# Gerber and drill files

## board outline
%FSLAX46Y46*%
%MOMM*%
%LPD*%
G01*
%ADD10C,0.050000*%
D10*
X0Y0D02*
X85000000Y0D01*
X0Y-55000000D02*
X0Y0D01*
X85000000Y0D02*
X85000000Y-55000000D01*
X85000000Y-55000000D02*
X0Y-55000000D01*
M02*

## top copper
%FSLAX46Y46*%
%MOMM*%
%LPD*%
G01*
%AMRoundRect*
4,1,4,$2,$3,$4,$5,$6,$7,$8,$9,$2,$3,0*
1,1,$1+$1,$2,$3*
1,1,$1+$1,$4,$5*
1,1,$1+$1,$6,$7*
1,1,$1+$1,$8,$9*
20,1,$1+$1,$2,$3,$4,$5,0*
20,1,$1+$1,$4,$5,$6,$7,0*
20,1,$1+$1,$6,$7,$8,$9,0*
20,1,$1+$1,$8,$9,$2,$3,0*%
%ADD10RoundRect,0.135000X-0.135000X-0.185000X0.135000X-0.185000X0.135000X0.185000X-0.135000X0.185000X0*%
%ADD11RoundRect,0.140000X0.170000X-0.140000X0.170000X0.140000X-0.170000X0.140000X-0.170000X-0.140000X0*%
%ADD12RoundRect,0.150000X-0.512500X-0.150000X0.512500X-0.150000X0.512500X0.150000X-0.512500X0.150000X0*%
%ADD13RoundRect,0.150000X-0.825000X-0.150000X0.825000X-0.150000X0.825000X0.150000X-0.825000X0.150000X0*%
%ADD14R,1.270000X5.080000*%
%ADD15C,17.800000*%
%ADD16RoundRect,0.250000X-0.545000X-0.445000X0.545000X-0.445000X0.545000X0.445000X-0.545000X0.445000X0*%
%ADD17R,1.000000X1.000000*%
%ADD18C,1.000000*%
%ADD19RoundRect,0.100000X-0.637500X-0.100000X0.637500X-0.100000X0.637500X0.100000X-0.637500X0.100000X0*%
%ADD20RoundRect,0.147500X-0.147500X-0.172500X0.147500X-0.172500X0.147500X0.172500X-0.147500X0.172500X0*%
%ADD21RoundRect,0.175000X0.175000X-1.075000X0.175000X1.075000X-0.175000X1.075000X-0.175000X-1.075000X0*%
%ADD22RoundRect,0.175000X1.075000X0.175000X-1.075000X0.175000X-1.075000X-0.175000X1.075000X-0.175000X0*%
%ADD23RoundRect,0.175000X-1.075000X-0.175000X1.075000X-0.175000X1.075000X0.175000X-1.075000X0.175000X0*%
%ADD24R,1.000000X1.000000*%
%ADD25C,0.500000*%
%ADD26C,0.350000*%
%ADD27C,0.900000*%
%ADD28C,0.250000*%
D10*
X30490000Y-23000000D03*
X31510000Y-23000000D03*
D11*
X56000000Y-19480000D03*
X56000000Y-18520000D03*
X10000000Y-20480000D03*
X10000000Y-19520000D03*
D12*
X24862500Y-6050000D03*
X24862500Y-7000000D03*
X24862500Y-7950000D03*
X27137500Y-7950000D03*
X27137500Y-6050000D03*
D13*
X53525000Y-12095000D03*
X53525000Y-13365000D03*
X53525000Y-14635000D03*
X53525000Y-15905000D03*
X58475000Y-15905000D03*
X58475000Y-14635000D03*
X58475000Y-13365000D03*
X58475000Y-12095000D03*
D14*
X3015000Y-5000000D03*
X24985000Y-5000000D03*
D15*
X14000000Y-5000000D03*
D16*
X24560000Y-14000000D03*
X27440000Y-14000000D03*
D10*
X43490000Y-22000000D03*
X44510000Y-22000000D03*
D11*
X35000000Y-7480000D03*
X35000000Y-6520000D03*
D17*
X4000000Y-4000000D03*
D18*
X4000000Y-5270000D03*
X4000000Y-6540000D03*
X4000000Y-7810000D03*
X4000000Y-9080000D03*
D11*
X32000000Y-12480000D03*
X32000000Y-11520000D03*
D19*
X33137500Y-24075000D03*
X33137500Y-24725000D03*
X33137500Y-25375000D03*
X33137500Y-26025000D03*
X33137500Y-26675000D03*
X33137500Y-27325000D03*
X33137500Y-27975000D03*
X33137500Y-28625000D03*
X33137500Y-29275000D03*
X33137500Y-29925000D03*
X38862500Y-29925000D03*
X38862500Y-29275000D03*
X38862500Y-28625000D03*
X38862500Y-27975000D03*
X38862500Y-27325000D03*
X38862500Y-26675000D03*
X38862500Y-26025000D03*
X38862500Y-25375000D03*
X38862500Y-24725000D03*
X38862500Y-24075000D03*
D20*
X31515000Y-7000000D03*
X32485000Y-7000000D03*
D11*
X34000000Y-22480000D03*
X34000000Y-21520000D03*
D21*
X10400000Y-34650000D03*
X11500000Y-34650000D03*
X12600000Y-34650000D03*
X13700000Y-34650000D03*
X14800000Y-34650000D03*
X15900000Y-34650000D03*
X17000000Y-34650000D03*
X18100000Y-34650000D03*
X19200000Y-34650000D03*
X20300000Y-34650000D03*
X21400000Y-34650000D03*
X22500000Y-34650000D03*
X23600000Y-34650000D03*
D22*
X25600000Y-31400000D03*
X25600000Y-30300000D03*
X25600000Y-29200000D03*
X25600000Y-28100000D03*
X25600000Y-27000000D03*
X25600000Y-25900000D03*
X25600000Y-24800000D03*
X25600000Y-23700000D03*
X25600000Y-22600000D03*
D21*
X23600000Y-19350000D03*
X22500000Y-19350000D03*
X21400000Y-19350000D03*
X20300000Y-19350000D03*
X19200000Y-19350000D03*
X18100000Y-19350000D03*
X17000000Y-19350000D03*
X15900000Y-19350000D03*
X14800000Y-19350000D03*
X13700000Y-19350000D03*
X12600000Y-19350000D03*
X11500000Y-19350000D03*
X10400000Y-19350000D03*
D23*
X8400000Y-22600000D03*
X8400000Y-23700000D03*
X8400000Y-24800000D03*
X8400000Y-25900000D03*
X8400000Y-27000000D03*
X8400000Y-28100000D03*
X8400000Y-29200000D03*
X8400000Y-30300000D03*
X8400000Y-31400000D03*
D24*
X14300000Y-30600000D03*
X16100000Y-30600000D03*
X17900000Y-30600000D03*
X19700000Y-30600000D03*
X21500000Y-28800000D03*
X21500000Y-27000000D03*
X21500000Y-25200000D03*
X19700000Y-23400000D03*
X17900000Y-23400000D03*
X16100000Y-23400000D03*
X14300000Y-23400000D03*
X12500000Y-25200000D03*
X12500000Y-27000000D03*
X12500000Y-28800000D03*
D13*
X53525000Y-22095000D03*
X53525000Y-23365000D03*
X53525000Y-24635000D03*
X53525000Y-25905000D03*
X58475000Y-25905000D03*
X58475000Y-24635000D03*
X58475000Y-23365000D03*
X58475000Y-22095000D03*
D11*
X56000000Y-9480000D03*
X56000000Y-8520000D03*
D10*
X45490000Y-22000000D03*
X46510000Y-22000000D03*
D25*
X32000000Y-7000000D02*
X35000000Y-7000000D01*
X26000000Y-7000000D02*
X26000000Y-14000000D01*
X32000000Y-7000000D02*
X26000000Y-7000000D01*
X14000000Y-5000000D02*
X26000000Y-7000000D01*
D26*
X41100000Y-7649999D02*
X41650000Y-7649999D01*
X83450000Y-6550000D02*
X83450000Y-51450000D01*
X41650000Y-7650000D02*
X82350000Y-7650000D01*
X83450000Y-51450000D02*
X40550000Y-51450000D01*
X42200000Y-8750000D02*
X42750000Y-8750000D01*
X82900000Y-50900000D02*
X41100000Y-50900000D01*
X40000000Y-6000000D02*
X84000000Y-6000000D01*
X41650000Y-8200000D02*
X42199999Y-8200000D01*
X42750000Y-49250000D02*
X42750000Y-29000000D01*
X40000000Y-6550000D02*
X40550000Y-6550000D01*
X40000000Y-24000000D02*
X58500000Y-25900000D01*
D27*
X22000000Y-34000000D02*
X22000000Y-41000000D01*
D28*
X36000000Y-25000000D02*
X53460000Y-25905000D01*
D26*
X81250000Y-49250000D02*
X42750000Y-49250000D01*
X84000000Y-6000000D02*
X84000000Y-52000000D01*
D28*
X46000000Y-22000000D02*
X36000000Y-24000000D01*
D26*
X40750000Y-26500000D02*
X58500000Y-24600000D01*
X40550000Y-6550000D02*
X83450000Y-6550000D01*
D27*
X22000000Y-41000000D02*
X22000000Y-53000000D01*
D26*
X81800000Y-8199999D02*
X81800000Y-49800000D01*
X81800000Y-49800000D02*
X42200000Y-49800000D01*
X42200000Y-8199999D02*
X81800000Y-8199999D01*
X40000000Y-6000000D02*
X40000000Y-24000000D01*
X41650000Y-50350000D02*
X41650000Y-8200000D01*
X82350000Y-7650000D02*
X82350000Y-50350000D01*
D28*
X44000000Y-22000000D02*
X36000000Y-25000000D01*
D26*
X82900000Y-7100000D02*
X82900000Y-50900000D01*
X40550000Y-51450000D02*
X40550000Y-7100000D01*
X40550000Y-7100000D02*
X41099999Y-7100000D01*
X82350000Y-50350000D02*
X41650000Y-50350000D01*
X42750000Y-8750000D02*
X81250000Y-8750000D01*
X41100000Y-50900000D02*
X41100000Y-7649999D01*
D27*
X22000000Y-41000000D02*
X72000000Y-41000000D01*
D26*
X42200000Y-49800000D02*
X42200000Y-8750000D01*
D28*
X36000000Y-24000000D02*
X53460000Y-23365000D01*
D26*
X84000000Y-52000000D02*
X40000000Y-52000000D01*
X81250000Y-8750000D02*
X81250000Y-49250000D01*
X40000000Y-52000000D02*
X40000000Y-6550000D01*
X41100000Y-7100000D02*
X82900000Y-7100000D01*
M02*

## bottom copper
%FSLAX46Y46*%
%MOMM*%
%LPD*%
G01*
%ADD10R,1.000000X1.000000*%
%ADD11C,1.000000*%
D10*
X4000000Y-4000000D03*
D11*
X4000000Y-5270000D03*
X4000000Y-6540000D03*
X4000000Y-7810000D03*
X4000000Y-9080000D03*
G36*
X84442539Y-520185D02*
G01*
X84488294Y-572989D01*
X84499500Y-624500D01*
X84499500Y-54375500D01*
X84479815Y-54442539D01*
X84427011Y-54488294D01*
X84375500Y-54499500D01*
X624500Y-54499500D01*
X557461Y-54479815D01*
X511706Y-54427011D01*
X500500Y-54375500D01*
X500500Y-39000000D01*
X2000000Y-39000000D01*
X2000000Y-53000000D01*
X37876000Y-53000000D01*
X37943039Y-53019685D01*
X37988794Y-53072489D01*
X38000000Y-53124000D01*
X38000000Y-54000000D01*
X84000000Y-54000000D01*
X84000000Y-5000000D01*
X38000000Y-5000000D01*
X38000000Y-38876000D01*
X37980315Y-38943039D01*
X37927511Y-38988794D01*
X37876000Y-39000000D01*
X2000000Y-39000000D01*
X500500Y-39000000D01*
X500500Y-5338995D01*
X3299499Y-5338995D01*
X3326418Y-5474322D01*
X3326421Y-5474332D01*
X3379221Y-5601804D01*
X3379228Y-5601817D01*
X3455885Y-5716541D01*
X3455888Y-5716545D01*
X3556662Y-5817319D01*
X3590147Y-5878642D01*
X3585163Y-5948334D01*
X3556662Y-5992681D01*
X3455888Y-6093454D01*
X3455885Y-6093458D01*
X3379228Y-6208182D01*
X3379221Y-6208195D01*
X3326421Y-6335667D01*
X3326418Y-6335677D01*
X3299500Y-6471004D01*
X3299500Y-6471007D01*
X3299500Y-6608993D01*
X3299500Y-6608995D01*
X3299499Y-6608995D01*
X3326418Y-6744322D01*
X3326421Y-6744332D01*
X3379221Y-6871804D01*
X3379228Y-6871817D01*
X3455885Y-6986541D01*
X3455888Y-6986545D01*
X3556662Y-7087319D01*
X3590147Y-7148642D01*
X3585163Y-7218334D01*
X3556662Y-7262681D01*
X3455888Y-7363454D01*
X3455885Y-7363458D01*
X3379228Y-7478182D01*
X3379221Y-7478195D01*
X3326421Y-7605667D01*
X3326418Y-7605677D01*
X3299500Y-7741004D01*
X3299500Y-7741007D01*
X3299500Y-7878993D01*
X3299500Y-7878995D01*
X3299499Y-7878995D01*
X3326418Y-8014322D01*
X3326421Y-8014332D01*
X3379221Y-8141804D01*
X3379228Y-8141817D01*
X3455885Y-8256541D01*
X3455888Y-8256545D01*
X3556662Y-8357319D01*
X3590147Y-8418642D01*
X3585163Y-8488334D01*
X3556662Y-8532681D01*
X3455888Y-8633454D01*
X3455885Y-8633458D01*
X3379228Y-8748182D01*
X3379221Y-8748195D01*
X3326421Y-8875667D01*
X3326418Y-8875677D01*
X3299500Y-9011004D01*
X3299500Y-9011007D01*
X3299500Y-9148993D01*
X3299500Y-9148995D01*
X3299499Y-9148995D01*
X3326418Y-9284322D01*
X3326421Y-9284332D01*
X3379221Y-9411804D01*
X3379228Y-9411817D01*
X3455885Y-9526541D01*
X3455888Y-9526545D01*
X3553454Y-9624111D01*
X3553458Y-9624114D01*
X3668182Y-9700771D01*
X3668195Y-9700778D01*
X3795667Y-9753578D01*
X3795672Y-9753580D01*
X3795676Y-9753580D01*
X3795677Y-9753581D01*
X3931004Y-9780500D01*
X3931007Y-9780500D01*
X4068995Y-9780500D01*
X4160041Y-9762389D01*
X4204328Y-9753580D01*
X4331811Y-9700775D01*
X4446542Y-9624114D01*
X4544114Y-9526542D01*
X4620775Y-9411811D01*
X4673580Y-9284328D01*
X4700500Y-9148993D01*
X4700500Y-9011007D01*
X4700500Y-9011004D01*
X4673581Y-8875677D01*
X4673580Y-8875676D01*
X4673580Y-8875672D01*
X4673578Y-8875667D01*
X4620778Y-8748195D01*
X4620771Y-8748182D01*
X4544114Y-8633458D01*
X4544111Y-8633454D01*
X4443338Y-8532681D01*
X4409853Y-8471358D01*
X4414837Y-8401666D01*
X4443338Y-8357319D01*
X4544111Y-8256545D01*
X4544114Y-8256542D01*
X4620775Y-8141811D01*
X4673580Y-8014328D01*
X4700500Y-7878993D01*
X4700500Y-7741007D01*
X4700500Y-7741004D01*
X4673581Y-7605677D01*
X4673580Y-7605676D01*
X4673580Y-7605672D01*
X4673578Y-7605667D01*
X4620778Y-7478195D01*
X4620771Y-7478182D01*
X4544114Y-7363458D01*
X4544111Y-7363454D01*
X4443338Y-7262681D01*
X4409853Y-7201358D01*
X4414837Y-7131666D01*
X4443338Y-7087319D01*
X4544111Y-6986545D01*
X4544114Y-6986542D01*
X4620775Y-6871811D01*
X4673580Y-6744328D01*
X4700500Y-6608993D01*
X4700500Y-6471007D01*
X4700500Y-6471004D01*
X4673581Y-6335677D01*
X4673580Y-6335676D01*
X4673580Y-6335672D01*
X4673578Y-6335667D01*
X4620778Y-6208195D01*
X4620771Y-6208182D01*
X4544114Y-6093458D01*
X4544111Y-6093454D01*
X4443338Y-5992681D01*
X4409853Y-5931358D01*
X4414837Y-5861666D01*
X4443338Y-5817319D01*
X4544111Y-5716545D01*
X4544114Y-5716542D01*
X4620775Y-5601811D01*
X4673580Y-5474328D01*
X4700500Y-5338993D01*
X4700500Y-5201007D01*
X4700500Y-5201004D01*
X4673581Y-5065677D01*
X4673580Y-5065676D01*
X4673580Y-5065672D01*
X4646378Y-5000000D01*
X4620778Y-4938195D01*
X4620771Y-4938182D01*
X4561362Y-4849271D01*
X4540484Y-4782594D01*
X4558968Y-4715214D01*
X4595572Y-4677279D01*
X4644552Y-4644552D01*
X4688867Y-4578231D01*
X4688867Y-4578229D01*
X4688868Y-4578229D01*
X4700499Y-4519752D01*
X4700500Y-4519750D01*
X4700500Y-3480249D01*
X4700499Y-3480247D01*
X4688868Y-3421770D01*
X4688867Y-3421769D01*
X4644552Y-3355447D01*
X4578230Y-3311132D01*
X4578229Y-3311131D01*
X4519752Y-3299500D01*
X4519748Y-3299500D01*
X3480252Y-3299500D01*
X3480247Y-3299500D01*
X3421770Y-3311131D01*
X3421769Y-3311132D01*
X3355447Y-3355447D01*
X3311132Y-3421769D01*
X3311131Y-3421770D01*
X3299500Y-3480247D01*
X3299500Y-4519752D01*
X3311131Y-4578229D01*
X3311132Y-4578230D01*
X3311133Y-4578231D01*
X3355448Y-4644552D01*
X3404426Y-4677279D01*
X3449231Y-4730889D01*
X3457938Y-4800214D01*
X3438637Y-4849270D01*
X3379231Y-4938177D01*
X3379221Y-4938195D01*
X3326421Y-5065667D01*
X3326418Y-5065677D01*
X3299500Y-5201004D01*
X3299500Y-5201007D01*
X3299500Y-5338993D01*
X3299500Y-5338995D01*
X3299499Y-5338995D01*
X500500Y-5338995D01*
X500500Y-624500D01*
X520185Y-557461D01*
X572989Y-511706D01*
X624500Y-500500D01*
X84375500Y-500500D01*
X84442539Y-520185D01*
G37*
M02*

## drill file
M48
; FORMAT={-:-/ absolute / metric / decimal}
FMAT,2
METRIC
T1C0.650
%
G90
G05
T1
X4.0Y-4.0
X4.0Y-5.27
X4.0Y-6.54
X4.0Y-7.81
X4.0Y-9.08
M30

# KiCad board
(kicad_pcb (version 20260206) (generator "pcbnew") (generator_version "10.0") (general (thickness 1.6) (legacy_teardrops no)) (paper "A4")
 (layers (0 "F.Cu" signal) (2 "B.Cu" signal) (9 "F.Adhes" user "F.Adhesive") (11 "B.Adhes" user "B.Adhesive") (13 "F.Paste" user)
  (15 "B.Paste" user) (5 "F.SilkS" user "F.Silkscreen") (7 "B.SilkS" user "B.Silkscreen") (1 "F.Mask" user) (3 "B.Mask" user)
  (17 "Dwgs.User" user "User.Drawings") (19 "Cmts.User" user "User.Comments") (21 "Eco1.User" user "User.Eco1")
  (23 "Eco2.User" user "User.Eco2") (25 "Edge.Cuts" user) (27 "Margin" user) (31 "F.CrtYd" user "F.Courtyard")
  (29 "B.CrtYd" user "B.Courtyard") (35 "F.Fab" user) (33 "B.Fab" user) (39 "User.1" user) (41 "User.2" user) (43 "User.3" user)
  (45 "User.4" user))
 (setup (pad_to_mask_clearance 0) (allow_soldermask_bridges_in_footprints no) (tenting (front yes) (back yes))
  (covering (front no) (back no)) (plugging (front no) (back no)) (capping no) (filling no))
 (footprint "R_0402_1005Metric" (layer "F.Cu") (at 31 23)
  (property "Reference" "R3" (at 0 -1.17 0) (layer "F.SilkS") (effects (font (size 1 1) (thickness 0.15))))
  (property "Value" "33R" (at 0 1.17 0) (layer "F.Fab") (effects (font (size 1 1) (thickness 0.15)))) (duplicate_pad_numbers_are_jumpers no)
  (pad "1" smd roundrect (at -0.51 0) (size 0.54 0.64) (layers "F.Cu" "F.Mask" "F.Paste") (roundrect_rratio 0.25))
  (pad "2" smd roundrect (at 0.51 0) (size 0.54 0.64) (layers "F.Cu" "F.Mask" "F.Paste") (roundrect_rratio 0.25)))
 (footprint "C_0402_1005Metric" (layer "F.Cu") (at 56 19 90)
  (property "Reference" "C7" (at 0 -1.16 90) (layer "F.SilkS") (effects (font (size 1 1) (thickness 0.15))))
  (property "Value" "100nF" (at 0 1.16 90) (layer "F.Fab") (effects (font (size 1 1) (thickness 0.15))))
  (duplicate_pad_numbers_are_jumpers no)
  (pad "1" smd roundrect (at -0.48 0 90) (size 0.56 0.62) (layers "F.Cu" "F.Mask" "F.Paste") (roundrect_rratio 0.25))
  (pad "2" smd roundrect (at 0.48 0 90) (size 0.56 0.62) (layers "F.Cu" "F.Mask" "F.Paste") (roundrect_rratio 0.25)))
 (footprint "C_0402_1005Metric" (layer "F.Cu") (at 10 20 90)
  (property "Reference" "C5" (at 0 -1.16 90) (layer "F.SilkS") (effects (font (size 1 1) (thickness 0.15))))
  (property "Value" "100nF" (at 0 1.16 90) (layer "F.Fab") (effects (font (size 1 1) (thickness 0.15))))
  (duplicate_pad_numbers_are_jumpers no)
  (pad "1" smd roundrect (at -0.48 0 90) (size 0.56 0.62) (layers "F.Cu" "F.Mask" "F.Paste") (roundrect_rratio 0.25))
  (pad "2" smd roundrect (at 0.48 0 90) (size 0.56 0.62) (layers "F.Cu" "F.Mask" "F.Paste") (roundrect_rratio 0.25)))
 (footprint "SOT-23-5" (layer "F.Cu") (at 26 7)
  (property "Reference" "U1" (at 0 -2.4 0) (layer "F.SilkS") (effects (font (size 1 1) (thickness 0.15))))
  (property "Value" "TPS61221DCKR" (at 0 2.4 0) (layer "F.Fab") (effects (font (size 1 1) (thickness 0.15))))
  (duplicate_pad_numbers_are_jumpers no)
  (pad "1" smd roundrect (at -1.1375 -0.95) (size 1.325 0.6) (layers "F.Cu" "F.Mask" "F.Paste") (roundrect_rratio 0.25))
  (pad "2" smd roundrect (at -1.1375 0) (size 1.325 0.6) (layers "F.Cu" "F.Mask" "F.Paste") (roundrect_rratio 0.25))
  (pad "3" smd roundrect (at -1.1375 0.95) (size 1.325 0.6) (layers "F.Cu" "F.Mask" "F.Paste") (roundrect_rratio 0.25))
  (pad "4" smd roundrect (at 1.1375 0.95) (size 1.325 0.6) (layers "F.Cu" "F.Mask" "F.Paste") (roundrect_rratio 0.25))
  (pad "5" smd roundrect (at 1.1375 -0.95) (size 1.325 0.6) (layers "F.Cu" "F.Mask" "F.Paste") (roundrect_rratio 0.25)))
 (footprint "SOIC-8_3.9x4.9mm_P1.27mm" (layer "F.Cu") (at 56 14)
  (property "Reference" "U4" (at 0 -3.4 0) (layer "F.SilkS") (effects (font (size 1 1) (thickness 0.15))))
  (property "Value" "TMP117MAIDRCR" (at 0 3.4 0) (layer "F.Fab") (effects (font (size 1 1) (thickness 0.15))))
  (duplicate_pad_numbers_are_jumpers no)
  (pad "1" smd roundrect (at -2.475 -1.905) (size 1.95 0.6) (layers "F.Cu" "F.Mask" "F.Paste") (roundrect_rratio 0.25))
  (pad "2" smd roundrect (at -2.475 -0.635) (size 1.95 0.6) (layers "F.Cu" "F.Mask" "F.Paste") (roundrect_rratio 0.25))
  (pad "3" smd roundrect (at -2.475 0.635) (size 1.95 0.6) (layers "F.Cu" "F.Mask" "F.Paste") (roundrect_rratio 0.25))
  (pad "4" smd roundrect (at -2.475 1.905) (size 1.95 0.6) (layers "F.Cu" "F.Mask" "F.Paste") (roundrect_rratio 0.25))
  (pad "5" smd roundrect (at 2.475 1.905) (size 1.95 0.6) (layers "F.Cu" "F.Mask" "F.Paste") (roundrect_rratio 0.25))
  (pad "6" smd roundrect (at 2.475 0.635) (size 1.95 0.6) (layers "F.Cu" "F.Mask" "F.Paste") (roundrect_rratio 0.25))
  (pad "7" smd roundrect (at 2.475 -0.635) (size 1.95 0.6) (layers "F.Cu" "F.Mask" "F.Paste") (roundrect_rratio 0.25))
  (pad "8" smd roundrect (at 2.475 -1.905) (size 1.95 0.6) (layers "F.Cu" "F.Mask" "F.Paste") (roundrect_rratio 0.25)))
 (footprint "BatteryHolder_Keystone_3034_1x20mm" (layer "F.Cu") (at 14 5)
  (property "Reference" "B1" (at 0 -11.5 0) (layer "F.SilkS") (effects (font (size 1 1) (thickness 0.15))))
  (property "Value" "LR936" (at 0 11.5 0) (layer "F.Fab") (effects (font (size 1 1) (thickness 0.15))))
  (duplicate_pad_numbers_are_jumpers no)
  (pad "1" smd rect (at -10.985 0) (size 1.27 5.08) (layers "F.Cu" "F.Mask" "F.Paste"))
  (pad "1" smd rect (at 10.985 0) (size 1.27 5.08) (layers "F.Cu" "F.Mask" "F.Paste"))
  (pad "2" smd circle (at 0 0) (size 17.8 17.8) (layers "F.Cu" "F.Mask")))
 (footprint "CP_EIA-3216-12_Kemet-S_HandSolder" (layer "F.Cu") (at 26 14)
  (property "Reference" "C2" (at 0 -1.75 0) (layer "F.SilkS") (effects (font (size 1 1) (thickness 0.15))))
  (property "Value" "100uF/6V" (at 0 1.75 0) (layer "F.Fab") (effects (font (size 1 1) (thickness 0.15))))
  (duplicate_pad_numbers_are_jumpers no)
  (pad "1" smd roundrect (at -1.44 0) (size 1.59 1.39) (layers "F.Cu" "F.Mask" "F.Paste") (roundrect_rratio 0.179856))
  (pad "2" smd roundrect (at 1.44 0) (size 1.59 1.39) (layers "F.Cu" "F.Mask" "F.Paste") (roundrect_rratio 0.179856)))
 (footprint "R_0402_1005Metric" (layer "F.Cu") (at 44 22)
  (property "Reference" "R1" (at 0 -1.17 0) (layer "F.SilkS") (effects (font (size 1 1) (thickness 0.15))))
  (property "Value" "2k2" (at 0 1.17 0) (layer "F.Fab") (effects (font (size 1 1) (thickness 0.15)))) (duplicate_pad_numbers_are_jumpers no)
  (pad "1" smd roundrect (at -0.51 0) (size 0.54 0.64) (layers "F.Cu" "F.Mask" "F.Paste") (roundrect_rratio 0.25))
  (pad "2" smd roundrect (at 0.51 0) (size 0.54 0.64) (layers "F.Cu" "F.Mask" "F.Paste") (roundrect_rratio 0.25)))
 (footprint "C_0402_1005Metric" (layer "F.Cu") (at 35 7 90)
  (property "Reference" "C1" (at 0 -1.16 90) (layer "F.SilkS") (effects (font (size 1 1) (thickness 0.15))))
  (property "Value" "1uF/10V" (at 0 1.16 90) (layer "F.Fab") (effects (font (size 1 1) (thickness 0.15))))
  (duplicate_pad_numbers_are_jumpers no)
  (pad "1" smd roundrect (at -0.48 0 90) (size 0.56 0.62) (layers "F.Cu" "F.Mask" "F.Paste") (roundrect_rratio 0.25))
  (pad "2" smd roundrect (at 0.48 0 90) (size 0.56 0.62) (layers "F.Cu" "F.Mask" "F.Paste") (roundrect_rratio 0.25)))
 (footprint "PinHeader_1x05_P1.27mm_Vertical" (layer "F.Cu") (at 4 4)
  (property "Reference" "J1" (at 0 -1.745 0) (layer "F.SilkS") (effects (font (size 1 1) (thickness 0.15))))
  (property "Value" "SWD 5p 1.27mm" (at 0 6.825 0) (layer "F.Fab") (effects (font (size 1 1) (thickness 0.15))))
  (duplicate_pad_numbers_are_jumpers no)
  (pad "1" thru_hole rect (at 0 0) (size 1 1) (drill 0.65) (layers "*.Cu" "*.Mask") (remove_unused_layers no))
  (pad "2" thru_hole circle (at 0 1.27) (size 1 1) (drill 0.65) (layers "*.Cu" "*.Mask") (remove_unused_layers no))
  (pad "3" thru_hole circle (at 0 2.54) (size 1 1) (drill 0.65) (layers "*.Cu" "*.Mask") (remove_unused_layers no))
  (pad "4" thru_hole circle (at 0 3.81) (size 1 1) (drill 0.65) (layers "*.Cu" "*.Mask") (remove_unused_layers no))
  (pad "5" thru_hole circle (at 0 5.08) (size 1 1) (drill 0.65) (layers "*.Cu" "*.Mask") (remove_unused_layers no)))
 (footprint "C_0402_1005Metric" (layer "F.Cu") (at 32 12 90)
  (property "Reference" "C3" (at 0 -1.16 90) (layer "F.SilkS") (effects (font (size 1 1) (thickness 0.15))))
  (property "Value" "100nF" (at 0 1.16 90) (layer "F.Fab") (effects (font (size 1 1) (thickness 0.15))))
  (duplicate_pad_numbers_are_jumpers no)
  (pad "1" smd roundrect (at -0.48 0 90) (size 0.56 0.62) (layers "F.Cu" "F.Mask" "F.Paste") (roundrect_rratio 0.25))
  (pad "2" smd roundrect (at 0.48 0 90) (size 0.56 0.62) (layers "F.Cu" "F.Mask" "F.Paste") (roundrect_rratio 0.25)))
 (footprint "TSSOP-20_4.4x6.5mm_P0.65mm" (layer "F.Cu") (at 36 27)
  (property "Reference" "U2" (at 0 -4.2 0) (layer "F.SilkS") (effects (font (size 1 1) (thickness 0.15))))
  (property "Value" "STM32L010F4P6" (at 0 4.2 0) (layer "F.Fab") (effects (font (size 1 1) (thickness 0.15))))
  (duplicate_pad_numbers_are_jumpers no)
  (pad "1" smd roundrect (at -2.8625 -2.925) (size 1.475 0.4) (layers "F.Cu" "F.Mask" "F.Paste") (roundrect_rratio 0.25))
  (pad "2" smd roundrect (at -2.8625 -2.275) (size 1.475 0.4) (layers "F.Cu" "F.Mask" "F.Paste") (roundrect_rratio 0.25))
  (pad "3" smd roundrect (at -2.8625 -1.625) (size 1.475 0.4) (layers "F.Cu" "F.Mask" "F.Paste") (roundrect_rratio 0.25))
  (pad "4" smd roundrect (at -2.8625 -0.975) (size 1.475 0.4) (layers "F.Cu" "F.Mask" "F.Paste") (roundrect_rratio 0.25))
  (pad "5" smd roundrect (at -2.8625 -0.325) (size 1.475 0.4) (layers "F.Cu" "F.Mask" "F.Paste") (roundrect_rratio 0.25))
  (pad "6" smd roundrect (at -2.8625 0.325) (size 1.475 0.4) (layers "F.Cu" "F.Mask" "F.Paste") (roundrect_rratio 0.25))
  (pad "7" smd roundrect (at -2.8625 0.975) (size 1.475 0.4) (layers "F.Cu" "F.Mask" "F.Paste") (roundrect_rratio 0.25))
  (pad "8" smd roundrect (at -2.8625 1.625) (size 1.475 0.4) (layers "F.Cu" "F.Mask" "F.Paste") (roundrect_rratio 0.25))
  (pad "9" smd roundrect (at -2.8625 2.275) (size 1.475 0.4) (layers "F.Cu" "F.Mask" "F.Paste") (roundrect_rratio 0.25))
  (pad "10" smd roundrect (at -2.8625 2.925) (size 1.475 0.4) (layers "F.Cu" "F.Mask" "F.Paste") (roundrect_rratio 0.25))
  (pad "11" smd roundrect (at 2.8625 2.925) (size 1.475 0.4) (layers "F.Cu" "F.Mask" "F.Paste") (roundrect_rratio 0.25))
  (pad "12" smd roundrect (at 2.8625 2.275) (size 1.475 0.4) (layers "F.Cu" "F.Mask" "F.Paste") (roundrect_rratio 0.25))
  (pad "13" smd roundrect (at 2.8625 1.625) (size 1.475 0.4) (layers "F.Cu" "F.Mask" "F.Paste") (roundrect_rratio 0.25))
  (pad "14" smd roundrect (at 2.8625 0.975) (size 1.475 0.4) (layers "F.Cu" "F.Mask" "F.Paste") (roundrect_rratio 0.25))
  (pad "15" smd roundrect (at 2.8625 0.325) (size 1.475 0.4) (layers "F.Cu" "F.Mask" "F.Paste") (roundrect_rratio 0.25))
  (pad "16" smd roundrect (at 2.8625 -0.325) (size 1.475 0.4) (layers "F.Cu" "F.Mask" "F.Paste") (roundrect_rratio 0.25))
  (pad "17" smd roundrect (at 2.8625 -0.975) (size 1.475 0.4) (layers "F.Cu" "F.Mask" "F.Paste") (roundrect_rratio 0.25))
  (pad "18" smd roundrect (at 2.8625 -1.625) (size 1.475 0.4) (layers "F.Cu" "F.Mask" "F.Paste") (roundrect_rratio 0.25))
  (pad "19" smd roundrect (at 2.8625 -2.275) (size 1.475 0.4) (layers "F.Cu" "F.Mask" "F.Paste") (roundrect_rratio 0.25))
  (pad "20" smd roundrect (at 2.8625 -2.925) (size 1.475 0.4) (layers "F.Cu" "F.Mask" "F.Paste") (roundrect_rratio 0.25)))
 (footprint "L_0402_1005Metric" (layer "F.Cu") (at 32 7)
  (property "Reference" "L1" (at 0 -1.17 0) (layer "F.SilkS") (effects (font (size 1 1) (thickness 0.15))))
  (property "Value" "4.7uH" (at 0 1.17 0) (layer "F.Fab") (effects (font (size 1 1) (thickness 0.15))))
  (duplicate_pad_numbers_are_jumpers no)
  (pad "1" smd roundrect (at -0.485 0) (size 0.59 0.64) (layers "F.Cu" "F.Mask" "F.Paste") (roundrect_rratio 0.25))
  (pad "2" smd roundrect (at 0.485 0) (size 0.59 0.64) (layers "F.Cu" "F.Mask" "F.Paste") (roundrect_rratio 0.25)))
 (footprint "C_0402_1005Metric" (layer "F.Cu") (at 34 22 90)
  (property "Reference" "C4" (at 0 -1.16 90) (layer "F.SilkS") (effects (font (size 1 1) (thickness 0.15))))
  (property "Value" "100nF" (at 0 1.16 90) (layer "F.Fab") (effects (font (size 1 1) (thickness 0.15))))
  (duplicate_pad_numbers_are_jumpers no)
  (pad "1" smd roundrect (at -0.48 0 90) (size 0.56 0.62) (layers "F.Cu" "F.Mask" "F.Paste") (roundrect_rratio 0.25))
  (pad "2" smd roundrect (at 0.48 0 90) (size 0.56 0.62) (layers "F.Cu" "F.Mask" "F.Paste") (roundrect_rratio 0.25)))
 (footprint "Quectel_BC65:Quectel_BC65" (layer "F.Cu") (at 17 27 90)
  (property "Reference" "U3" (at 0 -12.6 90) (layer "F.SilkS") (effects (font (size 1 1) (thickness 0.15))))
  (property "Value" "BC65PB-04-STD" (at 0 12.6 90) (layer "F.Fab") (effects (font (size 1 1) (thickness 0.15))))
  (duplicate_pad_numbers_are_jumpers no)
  (pad "" smd roundrect (at -8.05 -6.6 90) (size 2.9 0.595) (layers "F.Paste") (roundrect_rratio 0.25))
  (pad "" smd roundrect (at -8.05 -5.5 90) (size 2.9 0.595) (layers "F.Paste") (roundrect_rratio 0.25))
  (pad "" smd roundrect (at -8.05 -4.4 90) (size 2.9 0.595) (layers "F.Paste") (roundrect_rratio 0.25))
  (pad "" smd roundrect (at -8.05 -3.3 90) (size 2.9 0.595) (layers "F.Paste") (roundrect_rratio 0.25))
  (pad "" smd roundrect (at -8.05 -2.2 90) (size 2.9 0.595) (layers "F.Paste") (roundrect_rratio 0.25))
  (pad "" smd roundrect (at -8.05 -1.1 90) (size 2.9 0.595) (layers "F.Paste") (roundrect_rratio 0.25))
  (pad "" smd roundrect (at -8.05 0 90) (size 2.9 0.595) (layers "F.Paste") (roundrect_rratio 0.25))
  (pad "" smd roundrect (at -8.05 1.1 90) (size 2.9 0.595) (layers "F.Paste") (roundrect_rratio 0.25))
  (pad "" smd roundrect (at -8.05 2.2 90) (size 2.9 0.595) (layers "F.Paste") (roundrect_rratio 0.25))
  (pad "" smd roundrect (at -8.05 3.3 90) (size 2.9 0.595) (layers "F.Paste") (roundrect_rratio 0.25))
  (pad "" smd roundrect (at -8.05 4.4 90) (size 2.9 0.595) (layers "F.Paste") (roundrect_rratio 0.25))
  (pad "" smd roundrect (at -8.05 5.5 90) (size 2.9 0.595) (layers "F.Paste") (roundrect_rratio 0.25))
  (pad "" smd roundrect (at -8.05 6.6 90) (size 2.9 0.595) (layers "F.Paste") (roundrect_rratio 0.25))
  (pad "" smd roundrect (at -4.4 -9 180) (size 2.9 0.595) (layers "F.Paste") (roundrect_rratio 0.25))
  (pad "" smd roundrect (at -4.4 9 180) (size 2.9 0.595) (layers "F.Paste") (roundrect_rratio 0.25))
  (pad "" smd circle (at -3.6 -2.7 90) (size 0.9 0.9) (layers "F.Paste"))
  (pad "" smd circle (at -3.6 -0.9 90) (size 0.9 0.9) (layers "F.Paste"))
  (pad "" smd circle (at -3.6 0.9 90) (size 0.9 0.9) (layers "F.Paste"))
  (pad "" smd circle (at -3.6 2.7 90) (size 0.9 0.9) (layers "F.Paste"))
  (pad "" smd roundrect (at -3.3 -9 180) (size 2.9 0.595) (layers "F.Paste") (roundrect_rratio 0.25))
  (pad "" smd roundrect (at -3.3 9 180) (size 2.9 0.595) (layers "F.Paste") (roundrect_rratio 0.25))
  (pad "" smd roundrect (at -2.2 -9 180) (size 2.9 0.595) (layers "F.Paste") (roundrect_rratio 0.25))
  (pad "" smd roundrect (at -2.2 9 180) (size 2.9 0.595) (layers "F.Paste") (roundrect_rratio 0.25))
  (pad "" smd circle (at -1.8 -4.5 90) (size 0.9 0.9) (layers "F.Paste"))
  (pad "" smd circle (at -1.8 4.5 90) (size 0.9 0.9) (layers "F.Paste"))
  (pad "" smd roundrect (at -1.1 -9 180) (size 2.9 0.595) (layers "F.Paste") (roundrect_rratio 0.25))
  (pad "" smd roundrect (at -1.1 9 180) (size 2.9 0.595) (layers "F.Paste") (roundrect_rratio 0.25))
  (pad "" smd roundrect (at 0 -9 180) (size 2.9 0.595) (layers "F.Paste") (roundrect_rratio 0.25))
  (pad "" smd circle (at 0 -4.5 90) (size 0.9 0.9) (layers "F.Paste"))
  (pad "" smd circle (at 0 4.5 90) (size 0.9 0.9) (layers "F.Paste"))
  (pad "" smd roundrect (at 0 9 180) (size 2.9 0.595) (layers "F.Paste") (roundrect_rratio 0.25))
  (pad "" smd roundrect (at 1.1 -9 180) (size 2.9 0.595) (layers "F.Paste") (roundrect_rratio 0.25))
  (pad "" smd roundrect (at 1.1 9 180) (size 2.9 0.595) (layers "F.Paste") (roundrect_rratio 0.25))
  (pad "" smd circle (at 1.8 -4.5 90) (size 0.9 0.9) (layers "F.Paste"))
  (pad "" smd circle (at 1.8 4.5 90) (size 0.9 0.9) (layers "F.Paste"))
  (pad "" smd roundrect (at 2.2 -9 180) (size 2.9 0.595) (layers "F.Paste") (roundrect_rratio 0.25))
  (pad "" smd roundrect (at 2.2 9 180) (size 2.9 0.595) (layers "F.Paste") (roundrect_rratio 0.25))
  (pad "" smd roundrect (at 3.3 -9 180) (size 2.9 0.595) (layers "F.Paste") (roundrect_rratio 0.25))
  (pad "" smd roundrect (at 3.3 9 180) (size 2.9 0.595) (layers "F.Paste") (roundrect_rratio 0.25))
  (pad "" smd circle (at 3.6 -2.7 90) (size 0.9 0.9) (layers "F.Paste"))
  (pad "" smd circle (at 3.6 -0.9 90) (size 0.9 0.9) (layers "F.Paste"))
  (pad "" smd circle (at 3.6 0.9 90) (size 0.9 0.9) (layers "F.Paste"))
  (pad "" smd circle (at 3.6 2.7 90) (size 0.9 0.9) (layers "F.Paste"))
  (pad "" smd roundrect (at 4.4 -9 180) (size 2.9 0.595) (layers "F.Paste") (roundrect_rratio 0.25))
  (pad "" smd roundrect (at 4.4 9 180) (size 2.9 0.595) (layers "F.Paste") (roundrect_rratio 0.25))
  (pad "" smd roundrect (at 8.05 -6.6 90) (size 2.9 0.595) (layers "F.Paste") (roundrect_rratio 0.25))
  (pad "" smd roundrect (at 8.05 -5.5 90) (size 2.9 0.595) (layers "F.Paste") (roundrect_rratio 0.25))
  (pad "" smd roundrect (at 8.05 -4.4 90) (size 2.9 0.595) (layers "F.Paste") (roundrect_rratio 0.25))
  (pad "" smd roundrect (at 8.05 -3.3 90) (size 2.9 0.595) (layers "F.Paste") (roundrect_rratio 0.25))
  (pad "" smd roundrect (at 8.05 -2.2 90) (size 2.9 0.595) (layers "F.Paste") (roundrect_rratio 0.25))
  (pad "" smd roundrect (at 8.05 -1.1 90) (size 2.9 0.595) (layers "F.Paste") (roundrect_rratio 0.25))
  (pad "" smd roundrect (at 8.05 0 90) (size 2.9 0.595) (layers "F.Paste") (roundrect_rratio 0.25))
  (pad "" smd roundrect (at 8.05 1.1 90) (size 2.9 0.595) (layers "F.Paste") (roundrect_rratio 0.25))
  (pad "" smd roundrect (at 8.05 2.2 90) (size 2.9 0.595) (layers "F.Paste") (roundrect_rratio 0.25))
  (pad "" smd roundrect (at 8.05 3.3 90) (size 2.9 0.595) (layers "F.Paste") (roundrect_rratio 0.25))
  (pad "" smd roundrect (at 8.05 4.4 90) (size 2.9 0.595) (layers "F.Paste") (roundrect_rratio 0.25))
  (pad "" smd roundrect (at 8.05 5.5 90) (size 2.9 0.595) (layers "F.Paste") (roundrect_rratio 0.25))
  (pad "" smd roundrect (at 8.05 6.6 90) (size 2.9 0.595) (layers "F.Paste") (roundrect_rratio 0.25))
  (pad "1" smd roundrect (at -7.65 -6.6 90) (size 2.5 0.7) (layers "F.Cu" "F.Mask") (roundrect_rratio 0.25))
  (pad "2" smd roundrect (at -7.65 -5.5 90) (size 2.5 0.7) (layers "F.Cu" "F.Mask") (roundrect_rratio 0.25))
  (pad "3" smd roundrect (at -7.65 -4.4 90) (size 2.5 0.7) (layers "F.Cu" "F.Mask") (roundrect_rratio 0.25))
  (pad "4" smd roundrect (at -7.65 -3.3 90) (size 2.5 0.7) (layers "F.Cu" "F.Mask") (roundrect_rratio 0.25))
  (pad "5" smd roundrect (at -7.65 -2.2 90) (size 2.5 0.7) (layers "F.Cu" "F.Mask") (roundrect_rratio 0.25))
  (pad "6" smd roundrect (at -7.65 -1.1 90) (size 2.5 0.7) (layers "F.Cu" "F.Mask") (roundrect_rratio 0.25))
  (pad "7" smd roundrect (at -7.65 0 90) (size 2.5 0.7) (layers "F.Cu" "F.Mask") (roundrect_rratio 0.25))
  (pad "8" smd roundrect (at -7.65 1.1 90) (size 2.5 0.7) (layers "F.Cu" "F.Mask") (roundrect_rratio 0.25))
  (pad "9" smd roundrect (at -7.65 2.2 90) (size 2.5 0.7) (layers "F.Cu" "F.Mask") (roundrect_rratio 0.25))
  (pad "10" smd roundrect (at -7.65 3.3 90) (size 2.5 0.7) (layers "F.Cu" "F.Mask") (roundrect_rratio 0.25))
  (pad "11" smd roundrect (at -7.65 4.4 90) (size 2.5 0.7) (layers "F.Cu" "F.Mask") (roundrect_rratio 0.25))
  (pad "12" smd roundrect (at -7.65 5.5 90) (size 2.5 0.7) (layers "F.Cu" "F.Mask") (roundrect_rratio 0.25))
  (pad "13" smd roundrect (at -7.65 6.6 90) (size 2.5 0.7) (layers "F.Cu" "F.Mask") (roundrect_rratio 0.25))
  (pad "14" smd roundrect (at -4.4 8.6 180) (size 2.5 0.7) (layers "F.Cu" "F.Mask") (roundrect_rratio 0.25))
  (pad "15" smd roundrect (at -3.3 8.6 180) (size 2.5 0.7) (layers "F.Cu" "F.Mask") (roundrect_rratio 0.25))
  (pad "16" smd roundrect (at -2.2 8.6 180) (size 2.5 0.7) (layers "F.Cu" "F.Mask") (roundrect_rratio 0.25))
  (pad "17" smd roundrect (at -1.1 8.6 180) (size 2.5 0.7) (layers "F.Cu" "F.Mask") (roundrect_rratio 0.25))
  (pad "18" smd roundrect (at 0 8.6 180) (size 2.5 0.7) (layers "F.Cu" "F.Mask") (roundrect_rratio 0.25))
  (pad "19" smd roundrect (at 1.1 8.6 180) (size 2.5 0.7) (layers "F.Cu" "F.Mask") (roundrect_rratio 0.25))
  (pad "20" smd roundrect (at 2.2 8.6 180) (size 2.5 0.7) (layers "F.Cu" "F.Mask") (roundrect_rratio 0.25))
  (pad "21" smd roundrect (at 3.3 8.6 180) (size 2.5 0.7) (layers "F.Cu" "F.Mask") (roundrect_rratio 0.25))
  (pad "22" smd roundrect (at 4.4 8.6 180) (size 2.5 0.7) (layers "F.Cu" "F.Mask") (roundrect_rratio 0.25))
  (pad "23" smd roundrect (at 7.65 6.6 90) (size 2.5 0.7) (layers "F.Cu" "F.Mask") (roundrect_rratio 0.25))
  (pad "24" smd roundrect (at 7.65 5.5 90) (size 2.5 0.7) (layers "F.Cu" "F.Mask") (roundrect_rratio 0.25))
  (pad "25" smd roundrect (at 7.65 4.4 90) (size 2.5 0.7) (layers "F.Cu" "F.Mask") (roundrect_rratio 0.25))
  (pad "26" smd roundrect (at 7.65 3.3 90) (size 2.5 0.7) (layers "F.Cu" "F.Mask") (roundrect_rratio 0.25))
  (pad "27" smd roundrect (at 7.65 2.2 90) (size 2.5 0.7) (layers "F.Cu" "F.Mask") (roundrect_rratio 0.25))
  (pad "28" smd roundrect (at 7.65 1.1 90) (size 2.5 0.7) (layers "F.Cu" "F.Mask") (roundrect_rratio 0.25))
  (pad "29" smd roundrect (at 7.65 0 90) (size 2.5 0.7) (layers "F.Cu" "F.Mask") (roundrect_rratio 0.25))
  (pad "30" smd roundrect (at 7.65 -1.1 90) (size 2.5 0.7) (layers "F.Cu" "F.Mask") (roundrect_rratio 0.25))
  (pad "31" smd roundrect (at 7.65 -2.2 90) (size 2.5 0.7) (layers "F.Cu" "F.Mask") (roundrect_rratio 0.25))
  (pad "32" smd roundrect (at 7.65 -3.3 90) (size 2.5 0.7) (layers "F.Cu" "F.Mask") (roundrect_rratio 0.25))
  (pad "33" smd roundrect (at 7.65 -4.4 90) (size 2.5 0.7) (layers "F.Cu" "F.Mask") (roundrect_rratio 0.25))
  (pad "34" smd roundrect (at 7.65 -5.5 90) (size 2.5 0.7) (layers "F.Cu" "F.Mask") (roundrect_rratio 0.25))
  (pad "35" smd roundrect (at 7.65 -6.6 90) (size 2.5 0.7) (layers "F.Cu" "F.Mask") (roundrect_rratio 0.25))
  (pad "36" smd roundrect (at 4.4 -8.6) (size 2.5 0.7) (layers "F.Cu" "F.Mask") (roundrect_rratio 0.25))
  (pad "37" smd roundrect (at 3.3 -8.6) (size 2.5 0.7) (layers "F.Cu" "F.Mask") (roundrect_rratio 0.25))
  (pad "38" smd roundrect (at 2.2 -8.6) (size 2.5 0.7) (layers "F.Cu" "F.Mask") (roundrect_rratio 0.25))
  (pad "39" smd roundrect (at 1.1 -8.6) (size 2.5 0.7) (layers "F.Cu" "F.Mask") (roundrect_rratio 0.25))
  (pad "40" smd roundrect (at 0 -8.6) (size 2.5 0.7) (layers "F.Cu" "F.Mask") (roundrect_rratio 0.25))
  (pad "41" smd roundrect (at -1.1 -8.6) (size 2.5 0.7) (layers "F.Cu" "F.Mask") (roundrect_rratio 0.25))
  (pad "42" smd roundrect (at -2.2 -8.6) (size 2.5 0.7) (layers "F.Cu" "F.Mask") (roundrect_rratio 0.25))
  (pad "43" smd roundrect (at -3.3 -8.6) (size 2.5 0.7) (layers "F.Cu" "F.Mask") (roundrect_rratio 0.25))
  (pad "44" smd roundrect (at -4.4 -8.6) (size 2.5 0.7) (layers "F.Cu" "F.Mask") (roundrect_rratio 0.25))
  (pad "45" smd rect (at -3.6 -2.7 90) (size 1 1) (layers "F.Cu" "F.Mask"))
  (pad "46" smd rect (at -3.6 -0.9 90) (size 1 1) (layers "F.Cu" "F.Mask"))
  (pad "47" smd rect (at -3.6 0.9 90) (size 1 1) (layers "F.Cu" "F.Mask"))
  (pad "48" smd rect (at -3.6 2.7 90) (size 1 1) (layers "F.Cu" "F.Mask"))
  (pad "49" smd rect (at -1.8 4.5 90) (size 1 1) (layers "F.Cu" "F.Mask"))
  (pad "50" smd rect (at 0 4.5 90) (size 1 1) (layers "F.Cu" "F.Mask"))
  (pad "51" smd rect (at 1.8 4.5 90) (size 1 1) (layers "F.Cu" "F.Mask"))
  (pad "52" smd rect (at 3.6 2.7 90) (size 1 1) (layers "F.Cu" "F.Mask"))
  (pad "53" smd rect (at 3.6 0.9 90) (size 1 1) (layers "F.Cu" "F.Mask"))
  (pad "54" smd rect (at 3.6 -0.9 90) (size 1 1) (layers "F.Cu" "F.Mask"))
  (pad "55" smd rect (at 3.6 -2.7 90) (size 1 1) (layers "F.Cu" "F.Mask"))
  (pad "56" smd rect (at 1.8 -4.5 90) (size 1 1) (layers "F.Cu" "F.Mask"))
  (pad "57" smd rect (at 0 -4.5 90) (size 1 1) (layers "F.Cu" "F.Mask"))
  (pad "58" smd rect (at -1.8 -4.5 90) (size 1 1) (layers "F.Cu" "F.Mask")))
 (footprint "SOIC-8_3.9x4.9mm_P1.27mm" (layer "F.Cu") (at 56 24)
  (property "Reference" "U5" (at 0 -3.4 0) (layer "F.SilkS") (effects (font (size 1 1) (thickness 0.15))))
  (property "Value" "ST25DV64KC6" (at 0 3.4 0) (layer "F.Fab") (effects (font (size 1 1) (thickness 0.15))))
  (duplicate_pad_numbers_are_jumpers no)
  (pad "1" smd roundrect (at -2.475 -1.905) (size 1.95 0.6) (layers "F.Cu" "F.Mask" "F.Paste") (roundrect_rratio 0.25))
  (pad "2" smd roundrect (at -2.475 -0.635) (size 1.95 0.6) (layers "F.Cu" "F.Mask" "F.Paste") (roundrect_rratio 0.25))
  (pad "3" smd roundrect (at -2.475 0.635) (size 1.95 0.6) (layers "F.Cu" "F.Mask" "F.Paste") (roundrect_rratio 0.25))
  (pad "4" smd roundrect (at -2.475 1.905) (size 1.95 0.6) (layers "F.Cu" "F.Mask" "F.Paste") (roundrect_rratio 0.25))
  (pad "5" smd roundrect (at 2.475 1.905) (size 1.95 0.6) (layers "F.Cu" "F.Mask" "F.Paste") (roundrect_rratio 0.25))
  (pad "6" smd roundrect (at 2.475 0.635) (size 1.95 0.6) (layers "F.Cu" "F.Mask" "F.Paste") (roundrect_rratio 0.25))
  (pad "7" smd roundrect (at 2.475 -0.635) (size 1.95 0.6) (layers "F.Cu" "F.Mask" "F.Paste") (roundrect_rratio 0.25))
  (pad "8" smd roundrect (at 2.475 -1.905) (size 1.95 0.6) (layers "F.Cu" "F.Mask" "F.Paste") (roundrect_rratio 0.25)))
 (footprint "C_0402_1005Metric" (layer "F.Cu") (at 56 9 90)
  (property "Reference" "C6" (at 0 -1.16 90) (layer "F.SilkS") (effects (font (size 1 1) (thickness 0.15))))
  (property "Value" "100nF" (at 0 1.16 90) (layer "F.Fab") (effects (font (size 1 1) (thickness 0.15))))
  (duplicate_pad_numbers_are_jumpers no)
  (pad "1" smd roundrect (at -0.48 0 90) (size 0.56 0.62) (layers "F.Cu" "F.Mask" "F.Paste") (roundrect_rratio 0.25))
  (pad "2" smd roundrect (at 0.48 0 90) (size 0.56 0.62) (layers "F.Cu" "F.Mask" "F.Paste") (roundrect_rratio 0.25)))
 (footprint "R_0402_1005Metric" (layer "F.Cu") (at 46 22)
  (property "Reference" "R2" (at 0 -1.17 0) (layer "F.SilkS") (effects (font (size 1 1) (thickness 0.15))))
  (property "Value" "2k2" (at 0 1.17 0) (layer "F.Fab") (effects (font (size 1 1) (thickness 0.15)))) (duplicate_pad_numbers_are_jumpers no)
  (pad "1" smd roundrect (at -0.51 0) (size 0.54 0.64) (layers "F.Cu" "F.Mask" "F.Paste") (roundrect_rratio 0.25))
  (pad "2" smd roundrect (at 0.51 0) (size 0.54 0.64) (layers "F.Cu" "F.Mask" "F.Paste") (roundrect_rratio 0.25)))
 (gr_line (start 0 0) (end 85 0) (stroke (width 0.05) (type default)) (layer "Edge.Cuts"))
 (gr_line (start 0 55) (end 0 0) (stroke (width 0.05) (type default)) (layer "Edge.Cuts"))
 (gr_line (start 85 0) (end 85 55) (stroke (width 0.05) (type default)) (layer "Edge.Cuts"))
 (gr_line (start 85 55) (end 0 55) (stroke (width 0.05) (type default)) (layer "Edge.Cuts"))
 (segment (start 32 7) (end 35 7) (width 0.5) (layer "F.Cu") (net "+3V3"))
 (segment (start 26 7) (end 26 14) (width 0.5) (layer "F.Cu") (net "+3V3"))
 (segment (start 32 7) (end 26 7) (width 0.5) (layer "F.Cu") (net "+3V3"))
 (segment (start 14 5) (end 26 7) (width 0.5) (layer "F.Cu") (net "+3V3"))
 (segment (start 41.1 7.649999) (end 41.65 7.649999) (width 0.35) (layer "F.Cu") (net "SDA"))
 (segment (start 83.45 6.55) (end 83.45 51.45) (width 0.35) (layer "F.Cu") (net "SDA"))
 (segment (start 41.65 7.65) (end 82.35 7.65) (width 0.35) (layer "F.Cu") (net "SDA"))
 (segment (start 83.45 51.45) (end 40.55 51.45) (width 0.35) (layer "F.Cu") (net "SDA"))
 (segment (start 42.2 8.75) (end 42.75 8.75) (width 0.35) (layer "F.Cu") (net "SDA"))
 (segment (start 82.9 50.9) (end 41.1 50.9) (width 0.35) (layer "F.Cu") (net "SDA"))
 (segment (start 40 6) (end 84 6) (width 0.35) (layer "F.Cu") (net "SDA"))
 (segment (start 41.65 8.2) (end 42.199999 8.2) (width 0.35) (layer "F.Cu") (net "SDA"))
 (segment (start 42.75 49.25) (end 42.75 29) (width 0.35) (layer "F.Cu") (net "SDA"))
 (segment (start 40 6.55) (end 40.55 6.55) (width 0.35) (layer "F.Cu") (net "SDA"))
 (segment (start 40 24) (end 58.5 25.9) (width 0.35) (layer "F.Cu") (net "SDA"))
 (segment (start 22 34) (end 22 41) (width 0.9) (layer "F.Cu") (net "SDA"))
 (segment (start 36 25) (end 53.46 25.905) (width 0.25) (layer "F.Cu") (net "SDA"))
 (segment (start 81.25 49.25) (end 42.75 49.25) (width 0.35) (layer "F.Cu") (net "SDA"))
 (segment (start 84 6) (end 84 52) (width 0.35) (layer "F.Cu") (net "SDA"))
 (segment (start 46 22) (end 36 24) (width 0.25) (layer "F.Cu") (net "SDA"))
 (segment (start 40.75 26.5) (end 58.5 24.6) (width 0.35) (layer "F.Cu") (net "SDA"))
 (segment (start 40.55 6.55) (end 83.45 6.55) (width 0.35) (layer "F.Cu") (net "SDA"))
 (segment (start 22 41) (end 22 53) (width 0.9) (layer "F.Cu") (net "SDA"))
 (segment (start 81.8 8.199999) (end 81.8 49.8) (width 0.35) (layer "F.Cu") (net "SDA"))
 (segment (start 81.8 49.8) (end 42.2 49.8) (width 0.35) (layer "F.Cu") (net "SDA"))
 (segment (start 42.2 8.199999) (end 81.8 8.199999) (width 0.35) (layer "F.Cu") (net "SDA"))
 (segment (start 40 6) (end 40 24) (width 0.35) (layer "F.Cu") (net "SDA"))
 (segment (start 41.65 50.35) (end 41.65 8.2) (width 0.35) (layer "F.Cu") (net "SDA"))
 (segment (start 82.35 7.65) (end 82.35 50.35) (width 0.35) (layer "F.Cu") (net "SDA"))
 (segment (start 44 22) (end 36 25) (width 0.25) (layer "F.Cu") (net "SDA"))
 (segment (start 82.9 7.1) (end 82.9 50.9) (width 0.35) (layer "F.Cu") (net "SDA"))
 (segment (start 40.55 51.45) (end 40.55 7.1) (width 0.35) (layer "F.Cu") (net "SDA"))
 (segment (start 40.55 7.1) (end 41.099999 7.1) (width 0.35) (layer "F.Cu") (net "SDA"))
 (segment (start 82.35 50.35) (end 41.65 50.35) (width 0.35) (layer "F.Cu") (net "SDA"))
 (segment (start 42.75 8.75) (end 81.25 8.75) (width 0.35) (layer "F.Cu") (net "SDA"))
 (segment (start 41.1 50.9) (end 41.1 7.649999) (width 0.35) (layer "F.Cu") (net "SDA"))
 (segment (start 22 41) (end 72 41) (width 0.9) (layer "F.Cu") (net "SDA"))
 (segment (start 42.2 49.8) (end 42.2 8.75) (width 0.35) (layer "F.Cu") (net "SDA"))
 (segment (start 36 24) (end 53.46 23.365) (width 0.25) (layer "F.Cu") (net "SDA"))
 (segment (start 84 52) (end 40 52) (width 0.35) (layer "F.Cu") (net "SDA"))
 (segment (start 81.25 8.75) (end 81.25 49.25) (width 0.35) (layer "F.Cu") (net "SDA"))
 (segment (start 40 52) (end 40 6.55) (width 0.35) (layer "F.Cu") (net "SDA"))
 (segment (start 41.1 7.1) (end 82.9 7.1) (width 0.35) (layer "F.Cu") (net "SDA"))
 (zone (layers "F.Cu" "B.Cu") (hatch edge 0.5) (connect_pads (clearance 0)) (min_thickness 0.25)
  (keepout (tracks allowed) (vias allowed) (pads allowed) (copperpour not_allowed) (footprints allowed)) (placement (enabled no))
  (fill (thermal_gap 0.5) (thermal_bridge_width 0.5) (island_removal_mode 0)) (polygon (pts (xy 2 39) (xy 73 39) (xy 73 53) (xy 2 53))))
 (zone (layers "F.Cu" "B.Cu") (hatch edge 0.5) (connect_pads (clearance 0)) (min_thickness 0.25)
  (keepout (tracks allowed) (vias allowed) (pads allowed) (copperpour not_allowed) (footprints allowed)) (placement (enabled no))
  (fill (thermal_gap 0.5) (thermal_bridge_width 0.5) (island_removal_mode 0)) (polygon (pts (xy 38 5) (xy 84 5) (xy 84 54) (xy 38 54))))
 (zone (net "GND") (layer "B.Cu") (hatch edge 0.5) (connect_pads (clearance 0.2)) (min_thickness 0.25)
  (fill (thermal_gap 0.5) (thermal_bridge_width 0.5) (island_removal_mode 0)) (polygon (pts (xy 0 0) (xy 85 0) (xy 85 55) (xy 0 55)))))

